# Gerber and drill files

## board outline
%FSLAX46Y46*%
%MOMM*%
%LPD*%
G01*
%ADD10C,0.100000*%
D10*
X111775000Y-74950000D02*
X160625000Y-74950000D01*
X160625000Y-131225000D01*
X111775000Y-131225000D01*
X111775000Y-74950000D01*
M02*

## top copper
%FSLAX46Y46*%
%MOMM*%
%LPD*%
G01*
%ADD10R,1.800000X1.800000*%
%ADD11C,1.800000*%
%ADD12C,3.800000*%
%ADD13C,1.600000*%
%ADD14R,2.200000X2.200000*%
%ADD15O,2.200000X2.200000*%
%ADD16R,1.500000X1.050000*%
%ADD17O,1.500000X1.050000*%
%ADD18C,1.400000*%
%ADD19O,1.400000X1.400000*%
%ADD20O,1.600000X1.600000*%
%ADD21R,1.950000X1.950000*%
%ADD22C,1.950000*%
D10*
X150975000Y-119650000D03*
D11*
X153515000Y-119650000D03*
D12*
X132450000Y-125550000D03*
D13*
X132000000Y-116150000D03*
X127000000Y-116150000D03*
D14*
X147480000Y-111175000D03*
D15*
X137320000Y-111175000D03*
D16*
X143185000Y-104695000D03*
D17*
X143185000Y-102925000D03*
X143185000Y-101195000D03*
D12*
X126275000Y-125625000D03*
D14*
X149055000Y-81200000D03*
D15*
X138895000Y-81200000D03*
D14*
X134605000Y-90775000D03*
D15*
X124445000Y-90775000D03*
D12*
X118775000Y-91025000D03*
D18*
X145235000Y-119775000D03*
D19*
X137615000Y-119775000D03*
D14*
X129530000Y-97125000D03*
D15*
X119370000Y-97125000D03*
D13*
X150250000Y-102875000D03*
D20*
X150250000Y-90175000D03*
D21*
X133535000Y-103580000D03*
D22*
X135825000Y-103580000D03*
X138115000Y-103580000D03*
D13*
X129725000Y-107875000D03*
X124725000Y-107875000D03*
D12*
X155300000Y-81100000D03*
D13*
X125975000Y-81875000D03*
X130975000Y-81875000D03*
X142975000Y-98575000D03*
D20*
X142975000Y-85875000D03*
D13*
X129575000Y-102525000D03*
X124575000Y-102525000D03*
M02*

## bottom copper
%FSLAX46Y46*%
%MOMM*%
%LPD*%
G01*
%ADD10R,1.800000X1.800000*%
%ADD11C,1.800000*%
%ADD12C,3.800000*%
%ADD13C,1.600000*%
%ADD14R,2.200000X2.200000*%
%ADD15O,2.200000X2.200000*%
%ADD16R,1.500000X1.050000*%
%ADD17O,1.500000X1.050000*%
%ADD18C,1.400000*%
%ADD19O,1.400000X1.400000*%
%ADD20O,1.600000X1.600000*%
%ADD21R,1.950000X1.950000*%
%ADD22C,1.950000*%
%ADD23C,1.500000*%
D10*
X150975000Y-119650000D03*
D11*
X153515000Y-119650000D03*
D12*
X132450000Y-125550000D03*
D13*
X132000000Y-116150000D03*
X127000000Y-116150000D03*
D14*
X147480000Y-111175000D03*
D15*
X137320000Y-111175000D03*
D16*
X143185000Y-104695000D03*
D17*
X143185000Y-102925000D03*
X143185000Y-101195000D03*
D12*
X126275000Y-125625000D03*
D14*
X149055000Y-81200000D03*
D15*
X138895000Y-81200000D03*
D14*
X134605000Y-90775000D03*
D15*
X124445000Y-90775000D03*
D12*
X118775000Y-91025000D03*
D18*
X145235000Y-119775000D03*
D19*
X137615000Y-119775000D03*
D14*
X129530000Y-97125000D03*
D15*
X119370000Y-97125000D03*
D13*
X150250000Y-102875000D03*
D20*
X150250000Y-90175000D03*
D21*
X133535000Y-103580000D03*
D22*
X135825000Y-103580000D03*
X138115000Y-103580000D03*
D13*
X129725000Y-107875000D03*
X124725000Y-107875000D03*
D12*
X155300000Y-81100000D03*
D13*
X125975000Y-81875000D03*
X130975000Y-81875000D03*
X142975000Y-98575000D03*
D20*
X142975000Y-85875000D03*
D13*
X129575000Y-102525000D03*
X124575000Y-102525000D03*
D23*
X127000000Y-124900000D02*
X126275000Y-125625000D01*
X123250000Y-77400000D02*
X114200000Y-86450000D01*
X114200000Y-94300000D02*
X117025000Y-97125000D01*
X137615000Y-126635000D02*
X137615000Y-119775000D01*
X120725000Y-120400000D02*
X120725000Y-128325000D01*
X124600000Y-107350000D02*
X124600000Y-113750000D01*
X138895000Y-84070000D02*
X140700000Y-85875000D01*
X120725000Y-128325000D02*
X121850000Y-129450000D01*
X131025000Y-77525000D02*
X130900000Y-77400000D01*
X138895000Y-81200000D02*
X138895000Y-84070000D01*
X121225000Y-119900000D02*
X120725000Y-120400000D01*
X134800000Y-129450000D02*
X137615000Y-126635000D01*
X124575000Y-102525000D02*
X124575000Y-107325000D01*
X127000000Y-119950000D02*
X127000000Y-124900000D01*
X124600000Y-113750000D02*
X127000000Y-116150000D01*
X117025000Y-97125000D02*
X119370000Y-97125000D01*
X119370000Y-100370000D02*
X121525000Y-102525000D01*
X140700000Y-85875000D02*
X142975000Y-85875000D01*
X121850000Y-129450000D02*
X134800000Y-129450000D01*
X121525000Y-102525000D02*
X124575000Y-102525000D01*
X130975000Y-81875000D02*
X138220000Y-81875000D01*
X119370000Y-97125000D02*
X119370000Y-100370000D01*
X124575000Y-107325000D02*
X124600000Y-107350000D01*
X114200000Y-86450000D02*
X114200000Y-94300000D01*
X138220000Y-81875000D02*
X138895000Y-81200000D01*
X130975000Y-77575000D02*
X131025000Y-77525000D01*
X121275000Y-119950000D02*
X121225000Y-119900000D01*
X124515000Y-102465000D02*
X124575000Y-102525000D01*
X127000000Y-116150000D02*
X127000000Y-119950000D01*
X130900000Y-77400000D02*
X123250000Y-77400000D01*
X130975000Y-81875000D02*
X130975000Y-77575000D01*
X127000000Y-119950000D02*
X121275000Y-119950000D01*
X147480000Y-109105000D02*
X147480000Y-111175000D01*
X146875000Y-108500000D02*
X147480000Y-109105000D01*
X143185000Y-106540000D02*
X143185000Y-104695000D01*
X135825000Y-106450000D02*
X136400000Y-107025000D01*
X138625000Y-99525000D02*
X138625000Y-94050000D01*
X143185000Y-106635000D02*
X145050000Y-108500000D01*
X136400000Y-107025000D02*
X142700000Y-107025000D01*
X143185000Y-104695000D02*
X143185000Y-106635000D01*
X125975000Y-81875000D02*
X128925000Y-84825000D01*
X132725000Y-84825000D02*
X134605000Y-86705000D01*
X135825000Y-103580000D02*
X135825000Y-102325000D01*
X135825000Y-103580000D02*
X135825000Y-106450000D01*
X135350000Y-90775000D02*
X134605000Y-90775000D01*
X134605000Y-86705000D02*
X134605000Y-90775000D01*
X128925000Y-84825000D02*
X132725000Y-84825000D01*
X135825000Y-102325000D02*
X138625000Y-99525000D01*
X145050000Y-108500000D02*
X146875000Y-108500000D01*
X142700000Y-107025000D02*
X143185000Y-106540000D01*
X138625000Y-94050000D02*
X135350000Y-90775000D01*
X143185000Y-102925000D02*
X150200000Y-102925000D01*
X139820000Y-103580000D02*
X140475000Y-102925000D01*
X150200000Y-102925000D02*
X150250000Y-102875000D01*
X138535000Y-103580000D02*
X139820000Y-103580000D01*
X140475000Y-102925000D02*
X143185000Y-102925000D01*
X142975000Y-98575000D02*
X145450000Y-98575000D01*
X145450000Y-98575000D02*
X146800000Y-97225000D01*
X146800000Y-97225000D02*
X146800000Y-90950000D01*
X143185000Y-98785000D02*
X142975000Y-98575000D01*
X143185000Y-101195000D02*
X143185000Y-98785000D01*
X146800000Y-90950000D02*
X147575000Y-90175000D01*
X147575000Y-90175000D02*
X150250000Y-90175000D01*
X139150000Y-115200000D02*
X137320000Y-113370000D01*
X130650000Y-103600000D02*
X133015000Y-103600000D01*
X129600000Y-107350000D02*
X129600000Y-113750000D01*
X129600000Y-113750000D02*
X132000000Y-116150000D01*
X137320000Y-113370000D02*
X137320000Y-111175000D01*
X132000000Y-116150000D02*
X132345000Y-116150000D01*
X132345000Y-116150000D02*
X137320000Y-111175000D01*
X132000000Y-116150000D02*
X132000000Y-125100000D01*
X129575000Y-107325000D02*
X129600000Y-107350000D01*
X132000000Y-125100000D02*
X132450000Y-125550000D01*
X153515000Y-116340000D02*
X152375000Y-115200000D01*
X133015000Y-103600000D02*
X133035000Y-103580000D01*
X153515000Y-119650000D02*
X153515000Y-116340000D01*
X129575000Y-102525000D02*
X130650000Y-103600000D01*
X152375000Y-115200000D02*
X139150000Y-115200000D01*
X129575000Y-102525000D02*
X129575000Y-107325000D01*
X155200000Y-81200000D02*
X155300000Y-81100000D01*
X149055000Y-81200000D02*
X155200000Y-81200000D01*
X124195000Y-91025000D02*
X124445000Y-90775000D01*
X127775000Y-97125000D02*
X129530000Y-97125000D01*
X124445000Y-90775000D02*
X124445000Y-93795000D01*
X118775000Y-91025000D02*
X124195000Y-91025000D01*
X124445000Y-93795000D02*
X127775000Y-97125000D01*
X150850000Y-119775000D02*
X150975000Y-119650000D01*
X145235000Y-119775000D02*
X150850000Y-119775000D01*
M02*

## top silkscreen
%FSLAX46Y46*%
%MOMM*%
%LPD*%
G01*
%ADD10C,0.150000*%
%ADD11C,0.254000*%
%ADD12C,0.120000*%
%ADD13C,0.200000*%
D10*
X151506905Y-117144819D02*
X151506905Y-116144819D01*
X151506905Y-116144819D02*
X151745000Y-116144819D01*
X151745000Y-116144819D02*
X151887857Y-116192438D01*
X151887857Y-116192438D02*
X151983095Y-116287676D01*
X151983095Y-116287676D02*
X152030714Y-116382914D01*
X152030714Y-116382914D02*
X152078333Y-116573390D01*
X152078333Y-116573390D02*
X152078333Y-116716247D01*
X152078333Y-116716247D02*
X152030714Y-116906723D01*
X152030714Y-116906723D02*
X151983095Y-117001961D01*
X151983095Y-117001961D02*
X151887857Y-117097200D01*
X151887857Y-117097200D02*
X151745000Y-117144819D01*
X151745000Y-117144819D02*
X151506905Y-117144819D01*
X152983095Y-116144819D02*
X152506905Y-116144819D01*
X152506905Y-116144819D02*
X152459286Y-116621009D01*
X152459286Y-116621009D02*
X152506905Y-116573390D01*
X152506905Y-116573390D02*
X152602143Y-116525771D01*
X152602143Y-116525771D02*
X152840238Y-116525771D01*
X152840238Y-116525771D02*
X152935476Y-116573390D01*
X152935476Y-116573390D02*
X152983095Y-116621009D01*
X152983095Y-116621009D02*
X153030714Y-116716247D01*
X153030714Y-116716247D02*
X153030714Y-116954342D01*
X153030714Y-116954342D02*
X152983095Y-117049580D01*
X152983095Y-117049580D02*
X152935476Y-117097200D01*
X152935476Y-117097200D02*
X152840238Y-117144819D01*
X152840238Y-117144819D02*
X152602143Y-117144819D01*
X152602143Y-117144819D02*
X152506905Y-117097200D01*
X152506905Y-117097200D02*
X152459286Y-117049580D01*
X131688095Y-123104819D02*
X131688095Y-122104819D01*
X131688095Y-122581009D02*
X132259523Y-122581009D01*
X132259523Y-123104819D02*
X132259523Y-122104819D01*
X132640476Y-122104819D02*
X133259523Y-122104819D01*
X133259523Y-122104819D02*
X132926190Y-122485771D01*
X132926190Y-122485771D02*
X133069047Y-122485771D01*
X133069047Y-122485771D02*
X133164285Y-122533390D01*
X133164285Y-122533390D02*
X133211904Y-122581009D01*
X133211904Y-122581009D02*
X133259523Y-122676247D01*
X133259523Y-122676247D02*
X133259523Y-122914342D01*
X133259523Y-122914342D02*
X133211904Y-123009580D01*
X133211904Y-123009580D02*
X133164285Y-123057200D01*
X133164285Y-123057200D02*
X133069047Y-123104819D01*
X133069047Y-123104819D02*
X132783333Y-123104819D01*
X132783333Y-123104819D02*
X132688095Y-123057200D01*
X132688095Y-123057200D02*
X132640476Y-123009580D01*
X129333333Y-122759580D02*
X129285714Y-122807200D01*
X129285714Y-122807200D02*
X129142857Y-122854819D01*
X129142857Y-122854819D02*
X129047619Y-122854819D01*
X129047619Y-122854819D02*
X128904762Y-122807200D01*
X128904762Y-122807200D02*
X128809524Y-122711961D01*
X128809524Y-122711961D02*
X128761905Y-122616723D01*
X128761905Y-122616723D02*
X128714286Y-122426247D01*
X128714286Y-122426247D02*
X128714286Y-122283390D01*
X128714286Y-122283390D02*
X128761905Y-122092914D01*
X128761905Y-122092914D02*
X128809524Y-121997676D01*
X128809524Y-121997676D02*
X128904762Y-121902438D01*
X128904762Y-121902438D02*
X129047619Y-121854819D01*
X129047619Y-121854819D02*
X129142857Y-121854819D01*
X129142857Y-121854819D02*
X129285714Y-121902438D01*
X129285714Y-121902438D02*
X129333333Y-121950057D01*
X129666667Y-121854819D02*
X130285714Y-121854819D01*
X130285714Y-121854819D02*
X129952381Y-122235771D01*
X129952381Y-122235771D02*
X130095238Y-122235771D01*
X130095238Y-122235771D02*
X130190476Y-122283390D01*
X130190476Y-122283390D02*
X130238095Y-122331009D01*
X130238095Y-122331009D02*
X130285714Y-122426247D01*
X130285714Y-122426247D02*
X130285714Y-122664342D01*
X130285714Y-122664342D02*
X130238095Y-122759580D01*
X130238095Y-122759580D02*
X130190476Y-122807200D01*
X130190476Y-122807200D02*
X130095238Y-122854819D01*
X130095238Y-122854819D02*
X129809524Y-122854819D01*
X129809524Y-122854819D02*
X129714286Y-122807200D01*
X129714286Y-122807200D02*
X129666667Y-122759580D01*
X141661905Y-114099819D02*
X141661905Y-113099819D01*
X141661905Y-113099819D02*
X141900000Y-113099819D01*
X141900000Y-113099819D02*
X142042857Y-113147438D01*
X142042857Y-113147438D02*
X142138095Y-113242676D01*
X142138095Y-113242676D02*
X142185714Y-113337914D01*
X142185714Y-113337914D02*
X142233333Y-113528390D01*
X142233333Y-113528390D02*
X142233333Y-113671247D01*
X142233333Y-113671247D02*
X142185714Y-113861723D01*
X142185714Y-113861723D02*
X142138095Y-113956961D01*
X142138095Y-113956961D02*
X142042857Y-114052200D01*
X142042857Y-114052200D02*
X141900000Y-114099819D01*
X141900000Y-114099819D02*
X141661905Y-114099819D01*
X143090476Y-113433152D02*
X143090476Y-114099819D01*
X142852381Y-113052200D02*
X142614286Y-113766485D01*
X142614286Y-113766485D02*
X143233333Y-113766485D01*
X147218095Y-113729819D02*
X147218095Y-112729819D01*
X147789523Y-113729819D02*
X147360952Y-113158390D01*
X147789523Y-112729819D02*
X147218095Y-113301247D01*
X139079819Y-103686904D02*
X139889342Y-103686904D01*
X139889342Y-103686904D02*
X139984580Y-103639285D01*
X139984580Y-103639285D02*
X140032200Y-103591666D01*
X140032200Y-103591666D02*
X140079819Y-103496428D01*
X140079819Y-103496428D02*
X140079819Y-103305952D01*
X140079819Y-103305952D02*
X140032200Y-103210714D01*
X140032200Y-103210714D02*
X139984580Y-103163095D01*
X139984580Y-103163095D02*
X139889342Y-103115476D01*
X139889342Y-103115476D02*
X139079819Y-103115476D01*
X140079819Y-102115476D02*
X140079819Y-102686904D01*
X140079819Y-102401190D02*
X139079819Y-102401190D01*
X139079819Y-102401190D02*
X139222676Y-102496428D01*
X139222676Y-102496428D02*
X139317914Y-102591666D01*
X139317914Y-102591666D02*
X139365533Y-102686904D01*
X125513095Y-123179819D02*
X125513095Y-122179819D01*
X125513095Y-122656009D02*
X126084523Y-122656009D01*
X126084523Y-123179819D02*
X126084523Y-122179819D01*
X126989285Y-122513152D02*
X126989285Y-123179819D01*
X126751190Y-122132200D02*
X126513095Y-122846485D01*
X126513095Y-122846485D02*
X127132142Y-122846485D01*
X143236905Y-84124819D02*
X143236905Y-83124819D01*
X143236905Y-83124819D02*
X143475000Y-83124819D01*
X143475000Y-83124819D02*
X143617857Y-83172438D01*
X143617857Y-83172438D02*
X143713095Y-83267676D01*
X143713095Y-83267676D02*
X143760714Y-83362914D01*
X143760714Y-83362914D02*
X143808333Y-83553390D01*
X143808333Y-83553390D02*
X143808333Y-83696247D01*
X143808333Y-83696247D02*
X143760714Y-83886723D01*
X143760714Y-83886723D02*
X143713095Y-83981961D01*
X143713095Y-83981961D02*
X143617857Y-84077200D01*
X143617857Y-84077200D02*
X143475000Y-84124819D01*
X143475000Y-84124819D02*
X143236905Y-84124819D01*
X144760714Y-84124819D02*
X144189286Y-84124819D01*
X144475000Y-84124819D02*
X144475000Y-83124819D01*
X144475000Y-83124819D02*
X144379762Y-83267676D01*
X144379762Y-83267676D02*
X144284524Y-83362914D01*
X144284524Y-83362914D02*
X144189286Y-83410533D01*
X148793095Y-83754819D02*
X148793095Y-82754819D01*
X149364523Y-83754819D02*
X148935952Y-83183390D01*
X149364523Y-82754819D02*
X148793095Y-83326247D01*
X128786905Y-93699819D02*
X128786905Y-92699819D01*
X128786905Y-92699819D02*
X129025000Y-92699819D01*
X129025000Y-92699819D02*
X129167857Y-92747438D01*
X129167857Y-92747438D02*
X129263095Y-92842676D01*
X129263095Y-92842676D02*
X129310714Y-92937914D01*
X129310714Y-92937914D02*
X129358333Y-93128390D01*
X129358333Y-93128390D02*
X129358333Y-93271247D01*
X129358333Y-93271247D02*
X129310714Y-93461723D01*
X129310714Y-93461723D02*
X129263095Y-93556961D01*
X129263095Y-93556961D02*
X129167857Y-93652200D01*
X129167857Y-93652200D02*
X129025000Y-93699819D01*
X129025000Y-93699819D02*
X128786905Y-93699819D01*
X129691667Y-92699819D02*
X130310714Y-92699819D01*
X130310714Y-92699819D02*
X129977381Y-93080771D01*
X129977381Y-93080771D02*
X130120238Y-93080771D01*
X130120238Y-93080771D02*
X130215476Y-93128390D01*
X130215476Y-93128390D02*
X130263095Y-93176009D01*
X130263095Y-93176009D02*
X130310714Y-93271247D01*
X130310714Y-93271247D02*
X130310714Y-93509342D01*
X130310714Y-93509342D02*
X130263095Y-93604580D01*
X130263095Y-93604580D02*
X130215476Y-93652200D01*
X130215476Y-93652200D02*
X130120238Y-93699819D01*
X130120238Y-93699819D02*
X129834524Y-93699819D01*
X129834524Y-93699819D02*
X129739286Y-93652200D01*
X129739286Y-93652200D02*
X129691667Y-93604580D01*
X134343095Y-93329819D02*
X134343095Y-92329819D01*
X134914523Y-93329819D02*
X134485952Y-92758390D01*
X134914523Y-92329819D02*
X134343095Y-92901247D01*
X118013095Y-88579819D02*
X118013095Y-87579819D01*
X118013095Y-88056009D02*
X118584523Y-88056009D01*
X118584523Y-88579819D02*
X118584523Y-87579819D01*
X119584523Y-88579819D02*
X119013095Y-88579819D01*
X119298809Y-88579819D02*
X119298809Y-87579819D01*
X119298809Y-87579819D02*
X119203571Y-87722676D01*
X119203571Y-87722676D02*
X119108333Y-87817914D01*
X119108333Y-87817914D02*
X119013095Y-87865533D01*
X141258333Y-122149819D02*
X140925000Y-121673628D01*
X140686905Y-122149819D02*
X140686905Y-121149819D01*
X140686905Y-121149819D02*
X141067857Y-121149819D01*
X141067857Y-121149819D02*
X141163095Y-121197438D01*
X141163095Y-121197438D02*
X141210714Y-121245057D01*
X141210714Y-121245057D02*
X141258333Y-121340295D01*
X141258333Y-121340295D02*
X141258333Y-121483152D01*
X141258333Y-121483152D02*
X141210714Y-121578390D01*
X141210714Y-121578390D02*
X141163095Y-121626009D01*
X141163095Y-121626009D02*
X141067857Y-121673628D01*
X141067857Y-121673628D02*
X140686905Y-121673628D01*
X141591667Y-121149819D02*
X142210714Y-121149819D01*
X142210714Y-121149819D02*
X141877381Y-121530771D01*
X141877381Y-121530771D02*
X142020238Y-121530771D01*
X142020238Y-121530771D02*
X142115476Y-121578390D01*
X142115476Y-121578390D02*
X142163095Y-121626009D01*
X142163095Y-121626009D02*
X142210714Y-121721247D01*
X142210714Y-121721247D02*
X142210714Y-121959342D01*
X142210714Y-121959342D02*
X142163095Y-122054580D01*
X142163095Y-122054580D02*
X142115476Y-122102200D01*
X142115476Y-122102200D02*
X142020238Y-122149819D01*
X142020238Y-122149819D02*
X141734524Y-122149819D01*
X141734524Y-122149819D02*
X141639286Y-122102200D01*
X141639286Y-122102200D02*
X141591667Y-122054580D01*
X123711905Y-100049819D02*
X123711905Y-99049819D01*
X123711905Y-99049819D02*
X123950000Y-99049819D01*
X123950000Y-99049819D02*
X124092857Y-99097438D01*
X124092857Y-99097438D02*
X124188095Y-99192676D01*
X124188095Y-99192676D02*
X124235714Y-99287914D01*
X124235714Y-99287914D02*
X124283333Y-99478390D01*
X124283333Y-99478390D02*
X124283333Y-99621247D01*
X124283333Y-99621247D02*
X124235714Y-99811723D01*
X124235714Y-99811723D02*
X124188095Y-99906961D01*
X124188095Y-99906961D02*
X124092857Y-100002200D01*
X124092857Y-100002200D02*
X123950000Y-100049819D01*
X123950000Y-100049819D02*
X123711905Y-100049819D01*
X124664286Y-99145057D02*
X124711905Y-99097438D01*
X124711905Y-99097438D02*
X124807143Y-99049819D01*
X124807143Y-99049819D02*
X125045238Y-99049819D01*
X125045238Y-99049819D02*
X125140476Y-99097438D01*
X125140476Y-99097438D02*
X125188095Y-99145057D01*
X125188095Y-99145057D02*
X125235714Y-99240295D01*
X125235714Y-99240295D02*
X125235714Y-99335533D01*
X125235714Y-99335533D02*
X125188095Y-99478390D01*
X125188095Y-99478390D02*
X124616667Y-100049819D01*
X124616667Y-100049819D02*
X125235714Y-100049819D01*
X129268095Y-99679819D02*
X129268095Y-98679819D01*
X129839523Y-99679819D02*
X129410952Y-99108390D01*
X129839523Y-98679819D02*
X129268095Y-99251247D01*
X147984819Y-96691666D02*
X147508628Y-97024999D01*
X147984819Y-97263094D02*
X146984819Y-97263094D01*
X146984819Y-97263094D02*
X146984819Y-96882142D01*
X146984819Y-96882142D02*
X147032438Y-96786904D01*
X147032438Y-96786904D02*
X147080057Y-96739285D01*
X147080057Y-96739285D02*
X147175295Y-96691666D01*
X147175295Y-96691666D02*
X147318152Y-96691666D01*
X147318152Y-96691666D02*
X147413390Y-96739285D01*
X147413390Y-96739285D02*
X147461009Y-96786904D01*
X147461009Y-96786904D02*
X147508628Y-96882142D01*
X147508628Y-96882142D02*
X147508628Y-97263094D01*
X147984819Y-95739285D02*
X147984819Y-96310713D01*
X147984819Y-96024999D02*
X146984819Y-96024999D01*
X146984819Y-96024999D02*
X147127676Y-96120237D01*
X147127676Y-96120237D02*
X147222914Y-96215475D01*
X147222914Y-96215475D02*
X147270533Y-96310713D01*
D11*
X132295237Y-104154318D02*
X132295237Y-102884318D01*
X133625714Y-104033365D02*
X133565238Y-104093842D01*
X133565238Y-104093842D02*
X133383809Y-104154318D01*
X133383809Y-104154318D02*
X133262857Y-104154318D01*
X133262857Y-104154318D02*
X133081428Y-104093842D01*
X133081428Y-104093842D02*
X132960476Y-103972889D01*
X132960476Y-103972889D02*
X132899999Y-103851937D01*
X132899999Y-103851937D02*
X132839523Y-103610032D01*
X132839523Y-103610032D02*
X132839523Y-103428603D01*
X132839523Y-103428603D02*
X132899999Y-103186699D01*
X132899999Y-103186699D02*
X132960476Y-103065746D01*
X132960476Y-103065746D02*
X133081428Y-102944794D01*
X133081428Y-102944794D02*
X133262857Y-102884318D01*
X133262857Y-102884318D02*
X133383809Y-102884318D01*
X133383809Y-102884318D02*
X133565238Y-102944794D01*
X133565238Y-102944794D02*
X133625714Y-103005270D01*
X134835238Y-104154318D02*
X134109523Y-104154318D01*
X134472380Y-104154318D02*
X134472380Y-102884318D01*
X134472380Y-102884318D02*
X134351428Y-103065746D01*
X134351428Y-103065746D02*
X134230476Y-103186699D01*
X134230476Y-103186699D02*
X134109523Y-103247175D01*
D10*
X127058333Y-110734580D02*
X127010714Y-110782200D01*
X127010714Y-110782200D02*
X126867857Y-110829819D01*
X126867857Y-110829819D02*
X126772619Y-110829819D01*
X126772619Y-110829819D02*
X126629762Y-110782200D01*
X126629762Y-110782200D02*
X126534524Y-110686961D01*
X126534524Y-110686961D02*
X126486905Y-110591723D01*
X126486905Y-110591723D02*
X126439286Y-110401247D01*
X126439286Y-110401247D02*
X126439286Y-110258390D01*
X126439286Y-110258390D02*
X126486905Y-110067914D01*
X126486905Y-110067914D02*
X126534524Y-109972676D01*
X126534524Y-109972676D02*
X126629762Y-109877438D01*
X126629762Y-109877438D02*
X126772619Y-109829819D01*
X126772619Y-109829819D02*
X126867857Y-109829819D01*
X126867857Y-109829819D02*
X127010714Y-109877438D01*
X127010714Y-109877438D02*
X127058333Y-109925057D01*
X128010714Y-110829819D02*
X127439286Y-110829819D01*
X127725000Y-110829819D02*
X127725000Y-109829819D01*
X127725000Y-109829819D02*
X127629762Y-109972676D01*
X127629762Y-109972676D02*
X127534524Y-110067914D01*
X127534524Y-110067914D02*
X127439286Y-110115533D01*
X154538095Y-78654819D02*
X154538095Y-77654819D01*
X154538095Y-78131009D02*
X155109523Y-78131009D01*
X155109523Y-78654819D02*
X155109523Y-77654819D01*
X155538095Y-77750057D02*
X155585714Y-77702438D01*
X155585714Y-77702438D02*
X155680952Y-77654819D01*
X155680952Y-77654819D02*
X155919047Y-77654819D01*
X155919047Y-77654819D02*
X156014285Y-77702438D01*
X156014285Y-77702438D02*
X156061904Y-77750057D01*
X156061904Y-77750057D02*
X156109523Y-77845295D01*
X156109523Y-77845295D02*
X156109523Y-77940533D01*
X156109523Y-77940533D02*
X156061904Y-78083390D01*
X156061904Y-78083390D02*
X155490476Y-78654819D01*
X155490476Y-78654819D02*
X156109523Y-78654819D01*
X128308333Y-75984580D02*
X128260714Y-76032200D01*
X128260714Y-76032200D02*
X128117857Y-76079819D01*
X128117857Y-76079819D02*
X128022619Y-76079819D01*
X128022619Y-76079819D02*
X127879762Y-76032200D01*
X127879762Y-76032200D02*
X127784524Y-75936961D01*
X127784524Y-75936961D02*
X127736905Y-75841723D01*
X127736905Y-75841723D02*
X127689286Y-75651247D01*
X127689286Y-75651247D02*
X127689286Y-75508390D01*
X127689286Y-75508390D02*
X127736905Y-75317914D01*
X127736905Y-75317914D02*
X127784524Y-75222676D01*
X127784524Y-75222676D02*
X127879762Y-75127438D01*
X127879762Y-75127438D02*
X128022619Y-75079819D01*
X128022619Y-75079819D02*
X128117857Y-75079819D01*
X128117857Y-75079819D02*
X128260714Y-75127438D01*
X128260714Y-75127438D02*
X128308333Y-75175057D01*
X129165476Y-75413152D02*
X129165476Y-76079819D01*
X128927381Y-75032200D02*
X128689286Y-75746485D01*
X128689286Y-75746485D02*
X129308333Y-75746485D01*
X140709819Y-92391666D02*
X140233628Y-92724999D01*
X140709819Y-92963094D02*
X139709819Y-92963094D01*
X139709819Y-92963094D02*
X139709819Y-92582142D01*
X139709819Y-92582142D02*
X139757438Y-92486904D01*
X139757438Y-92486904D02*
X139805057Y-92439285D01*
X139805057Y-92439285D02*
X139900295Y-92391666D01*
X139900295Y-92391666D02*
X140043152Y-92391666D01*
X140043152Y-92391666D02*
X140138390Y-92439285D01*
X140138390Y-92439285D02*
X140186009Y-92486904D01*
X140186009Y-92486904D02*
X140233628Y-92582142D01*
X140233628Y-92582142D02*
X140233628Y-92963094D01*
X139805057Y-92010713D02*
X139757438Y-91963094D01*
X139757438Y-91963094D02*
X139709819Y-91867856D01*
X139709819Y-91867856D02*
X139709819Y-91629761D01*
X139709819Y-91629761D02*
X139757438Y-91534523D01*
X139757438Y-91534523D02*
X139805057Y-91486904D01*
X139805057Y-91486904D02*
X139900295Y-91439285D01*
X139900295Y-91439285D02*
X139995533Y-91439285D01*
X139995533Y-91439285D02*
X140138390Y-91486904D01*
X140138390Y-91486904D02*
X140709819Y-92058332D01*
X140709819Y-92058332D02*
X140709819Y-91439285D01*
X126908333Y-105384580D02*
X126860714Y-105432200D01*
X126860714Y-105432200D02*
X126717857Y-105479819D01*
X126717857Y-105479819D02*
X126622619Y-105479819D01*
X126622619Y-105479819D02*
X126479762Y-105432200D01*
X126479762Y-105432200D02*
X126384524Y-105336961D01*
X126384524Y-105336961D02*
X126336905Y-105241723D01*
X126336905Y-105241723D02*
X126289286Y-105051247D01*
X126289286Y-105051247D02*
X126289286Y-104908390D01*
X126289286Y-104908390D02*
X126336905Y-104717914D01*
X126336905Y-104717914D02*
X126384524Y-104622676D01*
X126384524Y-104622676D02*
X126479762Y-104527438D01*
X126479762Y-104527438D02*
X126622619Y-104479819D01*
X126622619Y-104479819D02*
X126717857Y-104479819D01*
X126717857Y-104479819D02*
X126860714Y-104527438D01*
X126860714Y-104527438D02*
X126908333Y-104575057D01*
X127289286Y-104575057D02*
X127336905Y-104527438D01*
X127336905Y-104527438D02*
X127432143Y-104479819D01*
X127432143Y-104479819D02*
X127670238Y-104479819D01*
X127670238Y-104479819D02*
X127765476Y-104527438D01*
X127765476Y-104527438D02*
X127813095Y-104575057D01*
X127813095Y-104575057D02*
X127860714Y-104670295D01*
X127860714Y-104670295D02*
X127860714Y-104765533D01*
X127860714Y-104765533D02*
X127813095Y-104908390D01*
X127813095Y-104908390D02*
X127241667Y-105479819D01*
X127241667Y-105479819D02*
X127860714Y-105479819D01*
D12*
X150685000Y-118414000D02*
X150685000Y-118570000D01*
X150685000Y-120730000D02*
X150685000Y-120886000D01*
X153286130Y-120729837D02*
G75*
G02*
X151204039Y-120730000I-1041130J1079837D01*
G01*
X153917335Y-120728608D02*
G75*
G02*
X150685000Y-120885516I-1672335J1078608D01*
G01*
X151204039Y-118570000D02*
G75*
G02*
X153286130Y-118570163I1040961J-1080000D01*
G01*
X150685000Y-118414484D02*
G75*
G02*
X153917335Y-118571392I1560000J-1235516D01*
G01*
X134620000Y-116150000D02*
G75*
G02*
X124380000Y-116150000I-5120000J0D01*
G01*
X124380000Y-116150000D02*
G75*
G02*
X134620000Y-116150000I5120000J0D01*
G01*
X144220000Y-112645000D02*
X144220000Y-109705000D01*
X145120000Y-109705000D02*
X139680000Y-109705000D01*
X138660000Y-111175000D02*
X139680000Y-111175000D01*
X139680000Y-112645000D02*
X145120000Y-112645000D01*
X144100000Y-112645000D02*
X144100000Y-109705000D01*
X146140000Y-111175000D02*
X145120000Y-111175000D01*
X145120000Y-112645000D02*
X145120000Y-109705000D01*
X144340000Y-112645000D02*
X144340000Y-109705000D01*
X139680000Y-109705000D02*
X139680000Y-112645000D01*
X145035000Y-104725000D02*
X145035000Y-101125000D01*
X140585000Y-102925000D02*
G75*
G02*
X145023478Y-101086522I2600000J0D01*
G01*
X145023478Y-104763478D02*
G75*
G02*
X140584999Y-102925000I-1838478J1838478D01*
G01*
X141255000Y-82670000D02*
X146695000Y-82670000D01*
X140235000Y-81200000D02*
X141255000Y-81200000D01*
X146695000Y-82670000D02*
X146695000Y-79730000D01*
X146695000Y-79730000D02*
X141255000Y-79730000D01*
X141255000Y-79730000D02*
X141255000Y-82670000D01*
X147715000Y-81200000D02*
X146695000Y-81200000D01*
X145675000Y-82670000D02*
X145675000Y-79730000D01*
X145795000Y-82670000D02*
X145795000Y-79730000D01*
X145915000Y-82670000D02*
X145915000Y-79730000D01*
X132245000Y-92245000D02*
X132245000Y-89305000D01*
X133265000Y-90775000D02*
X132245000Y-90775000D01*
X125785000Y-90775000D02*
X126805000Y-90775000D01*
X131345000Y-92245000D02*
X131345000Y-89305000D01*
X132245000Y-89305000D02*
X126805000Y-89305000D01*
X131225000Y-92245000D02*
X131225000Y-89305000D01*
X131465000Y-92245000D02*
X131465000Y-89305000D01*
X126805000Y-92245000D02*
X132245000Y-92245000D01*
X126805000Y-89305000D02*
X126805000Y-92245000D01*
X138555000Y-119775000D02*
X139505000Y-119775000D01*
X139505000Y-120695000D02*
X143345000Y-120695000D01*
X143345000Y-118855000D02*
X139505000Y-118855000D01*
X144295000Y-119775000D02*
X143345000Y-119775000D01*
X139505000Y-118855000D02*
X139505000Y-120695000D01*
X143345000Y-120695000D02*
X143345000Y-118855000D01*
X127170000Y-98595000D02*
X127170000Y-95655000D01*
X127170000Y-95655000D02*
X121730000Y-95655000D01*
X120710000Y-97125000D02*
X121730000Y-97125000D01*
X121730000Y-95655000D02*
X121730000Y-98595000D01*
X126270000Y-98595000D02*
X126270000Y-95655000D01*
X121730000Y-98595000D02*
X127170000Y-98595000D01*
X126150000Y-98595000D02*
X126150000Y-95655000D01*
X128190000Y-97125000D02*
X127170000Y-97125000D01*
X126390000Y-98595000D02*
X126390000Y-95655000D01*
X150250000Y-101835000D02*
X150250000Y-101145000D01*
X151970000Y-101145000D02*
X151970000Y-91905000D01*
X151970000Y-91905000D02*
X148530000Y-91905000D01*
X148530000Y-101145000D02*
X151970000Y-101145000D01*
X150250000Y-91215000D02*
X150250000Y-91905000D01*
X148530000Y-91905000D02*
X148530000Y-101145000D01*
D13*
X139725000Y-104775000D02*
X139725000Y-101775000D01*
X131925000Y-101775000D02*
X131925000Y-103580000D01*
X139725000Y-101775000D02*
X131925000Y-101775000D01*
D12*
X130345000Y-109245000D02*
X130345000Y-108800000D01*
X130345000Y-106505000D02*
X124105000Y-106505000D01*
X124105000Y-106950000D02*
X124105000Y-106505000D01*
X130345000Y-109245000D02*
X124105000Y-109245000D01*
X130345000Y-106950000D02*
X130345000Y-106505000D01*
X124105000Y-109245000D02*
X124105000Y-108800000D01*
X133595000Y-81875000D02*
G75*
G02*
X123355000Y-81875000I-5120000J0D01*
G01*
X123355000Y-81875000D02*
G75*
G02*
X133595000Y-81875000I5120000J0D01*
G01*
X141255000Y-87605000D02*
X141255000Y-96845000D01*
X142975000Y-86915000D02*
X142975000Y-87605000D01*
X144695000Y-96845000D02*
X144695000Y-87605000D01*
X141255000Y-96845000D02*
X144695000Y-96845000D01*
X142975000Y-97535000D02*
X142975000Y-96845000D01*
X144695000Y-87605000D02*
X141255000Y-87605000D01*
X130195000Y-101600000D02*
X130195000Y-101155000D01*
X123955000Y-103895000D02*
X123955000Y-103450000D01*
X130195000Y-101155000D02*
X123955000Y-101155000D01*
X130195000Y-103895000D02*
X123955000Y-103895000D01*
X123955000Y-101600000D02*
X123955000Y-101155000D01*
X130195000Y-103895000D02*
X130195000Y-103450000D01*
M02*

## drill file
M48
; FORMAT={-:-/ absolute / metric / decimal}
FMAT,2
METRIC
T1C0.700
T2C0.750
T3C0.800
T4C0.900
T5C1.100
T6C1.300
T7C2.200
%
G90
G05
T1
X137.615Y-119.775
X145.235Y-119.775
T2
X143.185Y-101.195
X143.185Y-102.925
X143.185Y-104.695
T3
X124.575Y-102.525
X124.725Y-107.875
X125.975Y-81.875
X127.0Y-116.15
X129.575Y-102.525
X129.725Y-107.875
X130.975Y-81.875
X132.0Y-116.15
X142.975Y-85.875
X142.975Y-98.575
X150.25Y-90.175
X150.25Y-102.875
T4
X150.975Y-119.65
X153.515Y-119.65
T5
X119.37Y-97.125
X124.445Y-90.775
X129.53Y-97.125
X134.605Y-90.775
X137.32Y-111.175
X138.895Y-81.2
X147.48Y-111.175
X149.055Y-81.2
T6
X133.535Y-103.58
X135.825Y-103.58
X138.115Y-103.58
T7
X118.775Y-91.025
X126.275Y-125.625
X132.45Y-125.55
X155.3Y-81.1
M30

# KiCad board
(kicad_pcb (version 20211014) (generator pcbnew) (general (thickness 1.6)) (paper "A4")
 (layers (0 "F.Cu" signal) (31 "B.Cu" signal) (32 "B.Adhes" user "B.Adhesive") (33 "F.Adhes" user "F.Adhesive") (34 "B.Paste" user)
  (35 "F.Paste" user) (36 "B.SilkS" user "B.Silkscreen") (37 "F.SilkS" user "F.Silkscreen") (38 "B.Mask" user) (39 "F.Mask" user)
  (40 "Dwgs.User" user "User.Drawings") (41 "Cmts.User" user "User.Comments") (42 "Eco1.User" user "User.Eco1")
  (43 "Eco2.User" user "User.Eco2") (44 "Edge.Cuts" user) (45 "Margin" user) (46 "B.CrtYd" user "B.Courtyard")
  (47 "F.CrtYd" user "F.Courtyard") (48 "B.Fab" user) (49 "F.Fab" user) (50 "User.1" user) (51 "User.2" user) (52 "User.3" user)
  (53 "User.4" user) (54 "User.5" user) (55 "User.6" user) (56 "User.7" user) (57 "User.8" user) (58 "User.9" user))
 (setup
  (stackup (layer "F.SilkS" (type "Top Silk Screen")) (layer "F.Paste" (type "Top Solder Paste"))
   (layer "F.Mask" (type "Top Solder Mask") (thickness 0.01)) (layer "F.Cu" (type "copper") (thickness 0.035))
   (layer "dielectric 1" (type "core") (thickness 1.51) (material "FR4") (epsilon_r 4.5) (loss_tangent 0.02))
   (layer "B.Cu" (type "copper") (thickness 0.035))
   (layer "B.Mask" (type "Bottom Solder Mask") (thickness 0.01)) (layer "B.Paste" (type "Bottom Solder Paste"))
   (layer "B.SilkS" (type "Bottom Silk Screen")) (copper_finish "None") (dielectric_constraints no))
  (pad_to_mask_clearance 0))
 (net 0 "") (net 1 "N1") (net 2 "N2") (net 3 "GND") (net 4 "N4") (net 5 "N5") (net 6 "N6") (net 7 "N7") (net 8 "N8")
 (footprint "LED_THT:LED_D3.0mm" (layer "F.Cu") (at 150.975 119.65)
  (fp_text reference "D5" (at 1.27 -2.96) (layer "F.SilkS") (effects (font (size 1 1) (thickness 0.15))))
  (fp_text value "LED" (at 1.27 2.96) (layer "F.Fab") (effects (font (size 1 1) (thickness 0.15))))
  (fp_line (start -0.29 -1.236) (end -0.29 -1.08) (layer "F.SilkS") (width 0.12))
  (fp_line (start -0.29 1.08) (end -0.29 1.236) (layer "F.SilkS") (width 0.12))
  (fp_arc (start 2.31113 1.079837) (mid 1.270117 1.5) (end 0.229039 1.08) (layer "F.SilkS") (width 0.12))
  (fp_arc (start 2.942335 1.078608) (mid 1.366487 1.987659) (end -0.29 1.235516) (layer "F.SilkS") (width 0.12))
  (fp_arc (start 0.229039 -1.08) (mid 1.270117 -1.5) (end 2.31113 -1.079837) (layer "F.SilkS") (width 0.12))
  (fp_arc (start -0.29 -1.235516) (mid 1.366487 -1.987659) (end 2.942335 -1.078608) (layer "F.SilkS") (width 0.12))
  (pad "1" thru_hole rect (at 0 0) (size 1.8 1.8) (drill 0.9) (layers *.Cu *.Mask) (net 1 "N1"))
  (pad "2" thru_hole circle (at 2.54 0) (size 1.8 1.8) (drill 0.9) (layers *.Cu *.Mask) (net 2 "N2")))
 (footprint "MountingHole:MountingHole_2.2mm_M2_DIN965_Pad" (layer "F.Cu") (at 132.45 125.55)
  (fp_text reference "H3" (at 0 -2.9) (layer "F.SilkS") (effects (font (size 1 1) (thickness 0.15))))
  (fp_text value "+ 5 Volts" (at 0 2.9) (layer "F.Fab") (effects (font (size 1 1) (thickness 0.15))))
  (pad "1" thru_hole circle (at 0 0) (size 3.8 3.8) (drill 2.2) (layers *.Cu *.Mask) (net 2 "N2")))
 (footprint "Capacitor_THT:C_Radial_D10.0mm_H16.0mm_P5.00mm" (layer "F.Cu") (at 132 116.15 180)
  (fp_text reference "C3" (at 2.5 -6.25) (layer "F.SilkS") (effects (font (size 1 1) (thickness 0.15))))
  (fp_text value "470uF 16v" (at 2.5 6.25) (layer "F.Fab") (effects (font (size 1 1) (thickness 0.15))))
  (fp_circle (center 2.5 0) (end 7.62 0) (layer "F.SilkS") (width 0.12) (fill none))
  (pad "1" thru_hole circle (at 0 0 180) (size 1.6 1.6) (drill 0.8) (layers *.Cu *.Mask) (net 2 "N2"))
  (pad "2" thru_hole circle (at 5 0 180) (size 1.6 1.6) (drill 0.8) (layers *.Cu *.Mask) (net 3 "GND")))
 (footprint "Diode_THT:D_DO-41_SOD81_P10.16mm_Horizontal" (layer "F.Cu") (at 147.48 111.175 180)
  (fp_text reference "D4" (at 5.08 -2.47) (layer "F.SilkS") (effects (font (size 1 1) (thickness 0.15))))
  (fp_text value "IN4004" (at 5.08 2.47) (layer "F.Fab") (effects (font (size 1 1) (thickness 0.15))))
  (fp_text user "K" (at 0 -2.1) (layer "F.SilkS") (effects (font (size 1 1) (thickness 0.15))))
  (fp_line (start 3.26 -1.47) (end 3.26 1.47) (layer "F.SilkS") (width 0.12))
  (fp_line (start 2.36 1.47) (end 7.8 1.47) (layer "F.SilkS") (width 0.12))
  (fp_line (start 8.82 0) (end 7.8 0) (layer "F.SilkS") (width 0.12))
  (fp_line (start 7.8 -1.47) (end 2.36 -1.47) (layer "F.SilkS") (width 0.12))
  (fp_line (start 3.38 -1.47) (end 3.38 1.47) (layer "F.SilkS") (width 0.12))
  (fp_line (start 1.34 0) (end 2.36 0) (layer "F.SilkS") (width 0.12))
  (fp_line (start 2.36 -1.47) (end 2.36 1.47) (layer "F.SilkS") (width 0.12))
  (fp_line (start 3.14 -1.47) (end 3.14 1.47) (layer "F.SilkS") (width 0.12))
  (fp_line (start 7.8 1.47) (end 7.8 -1.47) (layer "F.SilkS") (width 0.12))
  (pad "1" thru_hole rect (at 0 0 180) (size 2.2 2.2) (drill 1.1) (layers *.Cu *.Mask) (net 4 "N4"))
  (pad "2" thru_hole oval (at 10.16 0 180) (size 2.2 2.2) (drill 1.1) (layers *.Cu *.Mask) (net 2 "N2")))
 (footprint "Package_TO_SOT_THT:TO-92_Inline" (layer "F.Cu") (at 143.185 104.195 90)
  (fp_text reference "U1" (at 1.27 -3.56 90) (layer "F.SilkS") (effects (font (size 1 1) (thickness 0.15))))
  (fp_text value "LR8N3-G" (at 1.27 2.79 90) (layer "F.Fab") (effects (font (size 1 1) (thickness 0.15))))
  (fp_line (start -0.53 1.85) (end 3.07 1.85) (layer "F.SilkS") (width 0.12))
  (fp_arc (start 1.27 -2.6) (mid 3.672087 -0.994977) (end 3.108478 1.838478) (layer "F.SilkS") (width 0.12))
  (fp_arc (start -0.568478 1.838478) (mid -1.132087 -0.994977) (end 1.27 -2.6) (layer "F.SilkS") (width 0.12))
  (pad "1" thru_hole rect (at -0.5 0 90) (size 1.05 1.5) (drill 0.75) (layers *.Cu *.Mask) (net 4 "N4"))
  (pad "2" thru_hole oval (at 1.27 0 90) (size 1.05 1.5) (drill 0.75) (layers *.Cu *.Mask) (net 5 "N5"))
  (pad "3" thru_hole oval (at 3 0 90) (size 1.05 1.5) (drill 0.75) (layers *.Cu *.Mask) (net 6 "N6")))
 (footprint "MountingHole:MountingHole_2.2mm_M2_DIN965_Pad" (layer "F.Cu") (at 126.275 125.625)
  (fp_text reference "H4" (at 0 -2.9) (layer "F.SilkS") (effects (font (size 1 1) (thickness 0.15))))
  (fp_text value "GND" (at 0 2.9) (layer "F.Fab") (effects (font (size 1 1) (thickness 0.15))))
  (pad "1" thru_hole circle (at 0 0) (size 3.8 3.8) (drill 2.2) (layers *.Cu *.Mask) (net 3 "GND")))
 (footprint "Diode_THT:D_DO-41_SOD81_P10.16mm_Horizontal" (layer "F.Cu") (at 149.055 81.2 180)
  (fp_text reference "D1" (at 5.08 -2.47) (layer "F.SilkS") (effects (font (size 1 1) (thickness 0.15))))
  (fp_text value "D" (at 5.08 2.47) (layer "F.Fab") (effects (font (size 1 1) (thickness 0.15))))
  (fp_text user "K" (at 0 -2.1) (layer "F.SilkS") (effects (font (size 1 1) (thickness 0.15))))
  (fp_line (start 7.8 -1.47) (end 2.36 -1.47) (layer "F.SilkS") (width 0.12))
  (fp_line (start 8.82 0) (end 7.8 0) (layer "F.SilkS") (width 0.12))
  (fp_line (start 2.36 -1.47) (end 2.36 1.47) (layer "F.SilkS") (width 0.12))
  (fp_line (start 2.36 1.47) (end 7.8 1.47) (layer "F.SilkS") (width 0.12))
  (fp_line (start 7.8 1.47) (end 7.8 -1.47) (layer "F.SilkS") (width 0.12))
  (fp_line (start 1.34 0) (end 2.36 0) (layer "F.SilkS") (width 0.12))
  (fp_line (start 3.38 -1.47) (end 3.38 1.47) (layer "F.SilkS") (width 0.12))
  (fp_line (start 3.26 -1.47) (end 3.26 1.47) (layer "F.SilkS") (width 0.12))
  (fp_line (start 3.14 -1.47) (end 3.14 1.47) (layer "F.SilkS") (width 0.12))
  (pad "1" thru_hole rect (at 0 0 180) (size 2.2 2.2) (drill 1.1) (layers *.Cu *.Mask) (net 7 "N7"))
  (pad "2" thru_hole oval (at 10.16 0 180) (size 2.2 2.2) (drill 1.1) (layers *.Cu *.Mask) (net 3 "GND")))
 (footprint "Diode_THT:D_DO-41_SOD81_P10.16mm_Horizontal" (layer "F.Cu") (at 134.605 90.775 180)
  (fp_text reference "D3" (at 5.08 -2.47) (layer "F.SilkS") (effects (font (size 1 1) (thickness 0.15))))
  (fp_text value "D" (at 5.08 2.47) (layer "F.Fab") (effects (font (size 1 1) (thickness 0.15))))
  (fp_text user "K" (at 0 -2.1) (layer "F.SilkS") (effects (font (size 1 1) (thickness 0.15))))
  (fp_line (start 2.36 -1.47) (end 2.36 1.47) (layer "F.SilkS") (width 0.12))
  (fp_line (start 1.34 0) (end 2.36 0) (layer "F.SilkS") (width 0.12))
  (fp_line (start 8.82 0) (end 7.8 0) (layer "F.SilkS") (width 0.12))
  (fp_line (start 3.26 -1.47) (end 3.26 1.47) (layer "F.SilkS") (width 0.12))
  (fp_line (start 2.36 1.47) (end 7.8 1.47) (layer "F.SilkS") (width 0.12))
  (fp_line (start 3.38 -1.47) (end 3.38 1.47) (layer "F.SilkS") (width 0.12))
  (fp_line (start 3.14 -1.47) (end 3.14 1.47) (layer "F.SilkS") (width 0.12))
  (fp_line (start 7.8 -1.47) (end 2.36 -1.47) (layer "F.SilkS") (width 0.12))
  (fp_line (start 7.8 1.47) (end 7.8 -1.47) (layer "F.SilkS") (width 0.12))
  (pad "1" thru_hole rect (at 0 0 180) (size 2.2 2.2) (drill 1.1) (layers *.Cu *.Mask) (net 4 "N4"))
  (pad "2" thru_hole oval (at 10.16 0 180) (size 2.2 2.2) (drill 1.1) (layers *.Cu *.Mask) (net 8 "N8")))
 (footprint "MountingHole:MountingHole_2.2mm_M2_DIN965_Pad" (layer "F.Cu") (at 118.775 91.025)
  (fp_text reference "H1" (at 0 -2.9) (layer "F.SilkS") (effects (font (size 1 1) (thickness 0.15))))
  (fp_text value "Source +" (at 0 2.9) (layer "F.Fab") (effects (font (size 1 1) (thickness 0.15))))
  (pad "1" thru_hole circle (at 0 0) (size 3.8 3.8) (drill 2.2) (layers *.Cu *.Mask) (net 8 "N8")))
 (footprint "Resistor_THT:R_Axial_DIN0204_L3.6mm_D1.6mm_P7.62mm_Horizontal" (layer "F.Cu") (at 145.235 119.775 180)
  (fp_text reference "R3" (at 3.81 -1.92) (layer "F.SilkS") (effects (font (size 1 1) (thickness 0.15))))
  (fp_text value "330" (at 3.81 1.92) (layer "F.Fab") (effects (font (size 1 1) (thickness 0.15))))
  (fp_line (start 6.68 0) (end 5.73 0) (layer "F.SilkS") (width 0.12))
  (fp_line (start 5.73 -0.92) (end 1.89 -0.92) (layer "F.SilkS") (width 0.12))
  (fp_line (start 1.89 0.92) (end 5.73 0.92) (layer "F.SilkS") (width 0.12))
  (fp_line (start 0.94 0) (end 1.89 0) (layer "F.SilkS") (width 0.12))
  (fp_line (start 5.73 0.92) (end 5.73 -0.92) (layer "F.SilkS") (width 0.12))
  (fp_line (start 1.89 -0.92) (end 1.89 0.92) (layer "F.SilkS") (width 0.12))
  (pad "1" thru_hole circle (at 0 0 180) (size 1.4 1.4) (drill 0.7) (layers *.Cu *.Mask) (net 1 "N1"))
  (pad "2" thru_hole oval (at 7.62 0 180) (size 1.4 1.4) (drill 0.7) (layers *.Cu *.Mask) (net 3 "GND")))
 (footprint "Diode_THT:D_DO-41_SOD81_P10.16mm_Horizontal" (layer "F.Cu") (at 129.53 97.125 180)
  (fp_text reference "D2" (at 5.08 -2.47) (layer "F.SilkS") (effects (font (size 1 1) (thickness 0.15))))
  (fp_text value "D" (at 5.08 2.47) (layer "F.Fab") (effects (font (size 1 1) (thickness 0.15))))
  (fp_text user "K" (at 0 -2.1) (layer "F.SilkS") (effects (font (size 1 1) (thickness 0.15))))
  (fp_line (start 2.36 -1.47) (end 2.36 1.47) (layer "F.SilkS") (width 0.12))
  (fp_line (start 2.36 1.47) (end 7.8 1.47) (layer "F.SilkS") (width 0.12))
  (fp_line (start 8.82 0) (end 7.8 0) (layer "F.SilkS") (width 0.12))
  (fp_line (start 7.8 1.47) (end 7.8 -1.47) (layer "F.SilkS") (width 0.12))
  (fp_line (start 3.26 -1.47) (end 3.26 1.47) (layer "F.SilkS") (width 0.12))
  (fp_line (start 7.8 -1.47) (end 2.36 -1.47) (layer "F.SilkS") (width 0.12))
  (fp_line (start 3.38 -1.47) (end 3.38 1.47) (layer "F.SilkS") (width 0.12))
  (fp_line (start 1.34 0) (end 2.36 0) (layer "F.SilkS") (width 0.12))
  (fp_line (start 3.14 -1.47) (end 3.14 1.47) (layer "F.SilkS") (width 0.12))
  (pad "1" thru_hole rect (at 0 0 180) (size 2.2 2.2) (drill 1.1) (layers *.Cu *.Mask) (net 8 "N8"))
  (pad "2" thru_hole oval (at 10.16 0 180) (size 2.2 2.2) (drill 1.1) (layers *.Cu *.Mask) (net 3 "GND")))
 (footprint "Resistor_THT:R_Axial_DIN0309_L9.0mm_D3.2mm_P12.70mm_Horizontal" (layer "F.Cu") (at 150.25 102.875 90)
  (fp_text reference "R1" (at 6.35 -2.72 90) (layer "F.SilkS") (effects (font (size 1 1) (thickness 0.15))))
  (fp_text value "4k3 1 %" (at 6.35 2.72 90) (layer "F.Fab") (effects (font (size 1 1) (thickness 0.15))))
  (fp_line (start 1.04 0) (end 1.73 0) (layer "F.SilkS") (width 0.12))
  (fp_line (start 1.73 1.72) (end 10.97 1.72) (layer "F.SilkS") (width 0.12))
  (fp_line (start 10.97 1.72) (end 10.97 -1.72) (layer "F.SilkS") (width 0.12))
  (fp_line (start 1.73 -1.72) (end 1.73 1.72) (layer "F.SilkS") (width 0.12))
  (fp_line (start 11.66 0) (end 10.97 0) (layer "F.SilkS") (width 0.12))
  (fp_line (start 10.97 -1.72) (end 1.73 -1.72) (layer "F.SilkS") (width 0.12))
  (pad "1" thru_hole circle (at 0 0 90) (size 1.6 1.6) (drill 0.8) (layers *.Cu *.Mask) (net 5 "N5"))
  (pad "2" thru_hole oval (at 12.7 0 90) (size 1.6 1.6) (drill 0.8) (layers *.Cu *.Mask) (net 6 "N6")))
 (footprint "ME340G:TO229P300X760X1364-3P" (layer "F.Cu") (at 133.535 103.58)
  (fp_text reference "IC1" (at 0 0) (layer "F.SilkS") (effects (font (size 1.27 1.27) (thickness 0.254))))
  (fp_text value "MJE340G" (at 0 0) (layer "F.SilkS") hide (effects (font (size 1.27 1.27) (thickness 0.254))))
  (fp_line (start 6.19 1.195) (end 6.19 -1.805) (layer "F.SilkS") (width 0.2))
  (fp_line (start -1.61 -1.805) (end -1.61 0) (layer "F.SilkS") (width 0.2))
  (fp_line (start 6.19 -1.805) (end -1.61 -1.805) (layer "F.SilkS") (width 0.2))
  (pad "1" thru_hole rect locked (at 0 0) (size 1.95 1.95) (drill 1.3) (layers *.Cu *.Mask) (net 2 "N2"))
  (pad "2" thru_hole circle locked (at 2.29 0) (size 1.95 1.95) (drill 1.3) (layers *.Cu *.Mask) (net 4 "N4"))
  (pad "3" thru_hole circle locked (at 4.58 0) (size 1.95 1.95) (drill 1.3) (layers *.Cu *.Mask) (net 5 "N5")))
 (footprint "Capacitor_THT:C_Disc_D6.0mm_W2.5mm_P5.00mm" (layer "F.Cu") (at 129.725 107.875 180)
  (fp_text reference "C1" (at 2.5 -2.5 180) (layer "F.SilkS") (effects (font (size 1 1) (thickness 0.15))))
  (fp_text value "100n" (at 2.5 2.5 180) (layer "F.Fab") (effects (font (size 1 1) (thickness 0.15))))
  (fp_line (start -0.62 -1.37) (end -0.62 -0.925) (layer "F.SilkS") (width 0.12))
  (fp_line (start -0.62 1.37) (end 5.62 1.37) (layer "F.SilkS") (width 0.12))
  (fp_line (start 5.62 0.925) (end 5.62 1.37) (layer "F.SilkS") (width 0.12))
  (fp_line (start -0.62 -1.37) (end 5.62 -1.37) (layer "F.SilkS") (width 0.12))
  (fp_line (start -0.62 0.925) (end -0.62 1.37) (layer "F.SilkS") (width 0.12))
  (fp_line (start 5.62 -1.37) (end 5.62 -0.925) (layer "F.SilkS") (width 0.12))
  (pad "1" thru_hole circle (at 0 0 180) (size 1.6 1.6) (drill 0.8) (layers *.Cu *.Mask) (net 2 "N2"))
  (pad "2" thru_hole circle (at 5 0 180) (size 1.6 1.6) (drill 0.8) (layers *.Cu *.Mask) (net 3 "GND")))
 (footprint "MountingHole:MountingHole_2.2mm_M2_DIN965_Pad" (layer "F.Cu") (at 155.3 81.1)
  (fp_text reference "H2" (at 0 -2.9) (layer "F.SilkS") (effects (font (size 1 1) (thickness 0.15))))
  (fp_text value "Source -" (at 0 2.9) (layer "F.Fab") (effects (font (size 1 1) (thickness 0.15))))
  (pad "1" thru_hole circle (at 0 0) (size 3.8 3.8) (drill 2.2) (layers *.Cu *.Mask) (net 7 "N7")))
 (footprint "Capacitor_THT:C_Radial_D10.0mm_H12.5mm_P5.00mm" (layer "F.Cu") (at 125.975 81.875)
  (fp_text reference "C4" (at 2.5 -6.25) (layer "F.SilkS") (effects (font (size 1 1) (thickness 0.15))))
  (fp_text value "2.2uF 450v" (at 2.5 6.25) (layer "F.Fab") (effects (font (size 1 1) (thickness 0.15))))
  (fp_circle (center 2.5 0) (end 7.62 0) (layer "F.SilkS") (width 0.12) (fill none))
  (pad "1" thru_hole circle (at 0 0) (size 1.6 1.6) (drill 0.8) (layers *.Cu *.Mask) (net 4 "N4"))
  (pad "2" thru_hole circle (at 5 0) (size 1.6 1.6) (drill 0.8) (layers *.Cu *.Mask) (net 3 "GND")))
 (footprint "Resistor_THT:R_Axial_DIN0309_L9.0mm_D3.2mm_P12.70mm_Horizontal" (layer "F.Cu") (at 142.975 98.575 90)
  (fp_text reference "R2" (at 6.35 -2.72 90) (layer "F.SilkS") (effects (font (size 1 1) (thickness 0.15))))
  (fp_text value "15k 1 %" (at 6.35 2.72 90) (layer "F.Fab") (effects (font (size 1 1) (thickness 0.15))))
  (fp_line (start 10.97 -1.72) (end 1.73 -1.72) (layer "F.SilkS") (width 0.12))
  (fp_line (start 11.66 0) (end 10.97 0) (layer "F.SilkS") (width 0.12))
  (fp_line (start 1.73 1.72) (end 10.97 1.72) (layer "F.SilkS") (width 0.12))
  (fp_line (start 1.73 -1.72) (end 1.73 1.72) (layer "F.SilkS") (width 0.12))
  (fp_line (start 1.04 0) (end 1.73 0) (layer "F.SilkS") (width 0.12))
  (fp_line (start 10.97 1.72) (end 10.97 -1.72) (layer "F.SilkS") (width 0.12))
  (pad "1" thru_hole circle (at 0 0 90) (size 1.6 1.6) (drill 0.8) (layers *.Cu *.Mask) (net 6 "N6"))
  (pad "2" thru_hole oval (at 12.7 0 90) (size 1.6 1.6) (drill 0.8) (layers *.Cu *.Mask) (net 3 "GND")))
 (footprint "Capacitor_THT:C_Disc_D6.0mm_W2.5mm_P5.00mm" (layer "F.Cu") (at 129.575 102.525 180)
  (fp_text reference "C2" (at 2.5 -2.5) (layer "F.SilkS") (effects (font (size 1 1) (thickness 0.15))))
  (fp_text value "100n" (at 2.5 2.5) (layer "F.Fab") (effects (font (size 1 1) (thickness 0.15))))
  (fp_line (start -0.62 0.925) (end -0.62 1.37) (layer "F.SilkS") (width 0.12))
  (fp_line (start 5.62 -1.37) (end 5.62 -0.925) (layer "F.SilkS") (width 0.12))
  (fp_line (start -0.62 1.37) (end 5.62 1.37) (layer "F.SilkS") (width 0.12))
  (fp_line (start -0.62 -1.37) (end 5.62 -1.37) (layer "F.SilkS") (width 0.12))
  (fp_line (start 5.62 0.925) (end 5.62 1.37) (layer "F.SilkS") (width 0.12))
  (fp_line (start -0.62 -1.37) (end -0.62 -0.925) (layer "F.SilkS") (width 0.12))
  (pad "1" thru_hole circle (at 0 0 180) (size 1.6 1.6) (drill 0.8) (layers *.Cu *.Mask) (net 2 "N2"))
  (pad "2" thru_hole circle (at 5 0 180) (size 1.6 1.6) (drill 0.8) (layers *.Cu *.Mask) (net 3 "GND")))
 (gr_rect (start 111.775 74.95) (end 160.625 131.225) (layer "Edge.Cuts") (width 0.1) (fill none))
 (segment (start 127 124.9) (end 126.275 125.625) (width 1.5) (layer "B.Cu") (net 3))
 (segment (start 123.25 77.4) (end 114.2 86.45) (width 1.5) (layer "B.Cu") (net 3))
 (segment (start 114.2 94.3) (end 117.025 97.125) (width 1.5) (layer "B.Cu") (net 3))
 (segment (start 137.615 126.635) (end 137.615 119.775) (width 1.5) (layer "B.Cu") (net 3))
 (segment (start 120.725 120.4) (end 120.725 128.325) (width 1.5) (layer "B.Cu") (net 3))
 (segment (start 124.6 107.35) (end 124.6 113.75) (width 1.5) (layer "B.Cu") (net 3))
 (segment (start 138.895 84.07) (end 140.7 85.875) (width 1.5) (layer "B.Cu") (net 3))
 (segment (start 120.725 128.325) (end 121.85 129.45) (width 1.5) (layer "B.Cu") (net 3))
 (segment (start 131.025 77.525) (end 130.9 77.4) (width 1.5) (layer "B.Cu") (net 3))
 (segment (start 138.895 81.2) (end 138.895 84.07) (width 1.5) (layer "B.Cu") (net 3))
 (segment (start 121.225 119.9) (end 120.725 120.4) (width 1.5) (layer "B.Cu") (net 3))
 (segment (start 134.8 129.45) (end 137.615 126.635) (width 1.5) (layer "B.Cu") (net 3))
 (segment (start 124.575 102.525) (end 124.575 107.325) (width 1.5) (layer "B.Cu") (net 3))
 (segment (start 127 119.95) (end 127 124.9) (width 1.5) (layer "B.Cu") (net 3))
 (segment (start 124.6 113.75) (end 127 116.15) (width 1.5) (layer "B.Cu") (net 3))
 (segment (start 117.025 97.125) (end 119.37 97.125) (width 1.5) (layer "B.Cu") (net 3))
 (segment (start 119.37 100.37) (end 121.525 102.525) (width 1.5) (layer "B.Cu") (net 3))
 (segment (start 140.7 85.875) (end 142.975 85.875) (width 1.5) (layer "B.Cu") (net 3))
 (segment (start 121.85 129.45) (end 134.8 129.45) (width 1.5) (layer "B.Cu") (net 3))
 (segment (start 121.525 102.525) (end 124.575 102.525) (width 1.5) (layer "B.Cu") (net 3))
 (segment (start 130.975 81.875) (end 138.22 81.875) (width 1.5) (layer "B.Cu") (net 3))
 (segment (start 119.37 97.125) (end 119.37 100.37) (width 1.5) (layer "B.Cu") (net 3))
 (segment (start 124.575 107.325) (end 124.6 107.35) (width 1.5) (layer "B.Cu") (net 3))
 (segment (start 114.2 86.45) (end 114.2 94.3) (width 1.5) (layer "B.Cu") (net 3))
 (segment (start 138.22 81.875) (end 138.895 81.2) (width 1.5) (layer "B.Cu") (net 3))
 (segment (start 130.975 77.575) (end 131.025 77.525) (width 1.5) (layer "B.Cu") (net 3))
 (segment (start 121.275 119.95) (end 121.225 119.9) (width 1.5) (layer "B.Cu") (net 3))
 (segment (start 124.515 102.465) (end 124.575 102.525) (width 1.5) (layer "B.Cu") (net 3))
 (segment (start 127 116.15) (end 127 119.95) (width 1.5) (layer "B.Cu") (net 3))
 (segment (start 130.9 77.4) (end 123.25 77.4) (width 1.5) (layer "B.Cu") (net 3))
 (segment (start 130.975 81.875) (end 130.975 77.575) (width 1.5) (layer "B.Cu") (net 3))
 (segment (start 127 119.95) (end 121.275 119.95) (width 1.5) (layer "B.Cu") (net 3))
 (segment (start 147.48 109.105) (end 147.48 111.175) (width 1.5) (layer "B.Cu") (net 4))
 (segment (start 146.875 108.5) (end 147.48 109.105) (width 1.5) (layer "B.Cu") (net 4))
 (segment (start 143.185 106.54) (end 143.185 104.695) (width 1.5) (layer "B.Cu") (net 4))
 (segment (start 135.825 106.45) (end 136.4 107.025) (width 1.5) (layer "B.Cu") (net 4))
 (segment (start 138.625 99.525) (end 138.625 94.05) (width 1.5) (layer "B.Cu") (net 4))
 (segment (start 143.185 106.635) (end 145.05 108.5) (width 1.5) (layer "B.Cu") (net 4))
 (segment (start 136.4 107.025) (end 142.7 107.025) (width 1.5) (layer "B.Cu") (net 4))
 (segment (start 143.185 104.695) (end 143.185 106.635) (width 1.5) (layer "B.Cu") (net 4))
 (segment (start 125.975 81.875) (end 128.925 84.825) (width 1.5) (layer "B.Cu") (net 4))
 (segment (start 132.725 84.825) (end 134.605 86.705) (width 1.5) (layer "B.Cu") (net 4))
 (segment (start 135.825 103.58) (end 135.825 102.325) (width 1.5) (layer "B.Cu") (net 4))
 (segment (start 135.825 103.58) (end 135.825 106.45) (width 1.5) (layer "B.Cu") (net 4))
 (segment (start 135.35 90.775) (end 134.605 90.775) (width 1.5) (layer "B.Cu") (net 4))
 (segment (start 134.605 86.705) (end 134.605 90.775) (width 1.5) (layer "B.Cu") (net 4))
 (segment (start 128.925 84.825) (end 132.725 84.825) (width 1.5) (layer "B.Cu") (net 4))
 (segment (start 135.825 102.325) (end 138.625 99.525) (width 1.5) (layer "B.Cu") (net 4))
 (segment (start 145.05 108.5) (end 146.875 108.5) (width 1.5) (layer "B.Cu") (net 4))
 (segment (start 142.7 107.025) (end 143.185 106.54) (width 1.5) (layer "B.Cu") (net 4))
 (segment (start 138.625 94.05) (end 135.35 90.775) (width 1.5) (layer "B.Cu") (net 4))
 (segment (start 143.185 102.925) (end 150.2 102.925) (width 1.5) (layer "B.Cu") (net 5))
 (segment (start 139.82 103.58) (end 140.475 102.925) (width 1.5) (layer "B.Cu") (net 5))
 (segment (start 150.2 102.925) (end 150.25 102.875) (width 1.5) (layer "B.Cu") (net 5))
 (segment (start 138.535 103.58) (end 139.82 103.58) (width 1.5) (layer "B.Cu") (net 5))
 (segment (start 140.475 102.925) (end 143.185 102.925) (width 1.5) (layer "B.Cu") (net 5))
 (segment (start 142.975 98.575) (end 145.45 98.575) (width 1.5) (layer "B.Cu") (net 6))
 (segment (start 145.45 98.575) (end 146.8 97.225) (width 1.5) (layer "B.Cu") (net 6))
 (segment (start 146.8 97.225) (end 146.8 90.95) (width 1.5) (layer "B.Cu") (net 6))
 (segment (start 143.185 98.785) (end 142.975 98.575) (width 1.5) (layer "B.Cu") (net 6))
 (segment (start 143.185 101.195) (end 143.185 98.785) (width 1.5) (layer "B.Cu") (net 6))
 (segment (start 146.8 90.95) (end 147.575 90.175) (width 1.5) (layer "B.Cu") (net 6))
 (segment (start 147.575 90.175) (end 150.25 90.175) (width 1.5) (layer "B.Cu") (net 6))
 (segment (start 139.15 115.2) (end 137.32 113.37) (width 1.5) (layer "B.Cu") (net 2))
 (segment (start 130.65 103.6) (end 133.015 103.6) (width 1.5) (layer "B.Cu") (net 2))
 (segment (start 129.6 107.35) (end 129.6 113.75) (width 1.5) (layer "B.Cu") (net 2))
 (segment (start 129.6 113.75) (end 132 116.15) (width 1.5) (layer "B.Cu") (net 2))
 (segment (start 137.32 113.37) (end 137.32 111.175) (width 1.5) (layer "B.Cu") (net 2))
 (segment (start 132 116.15) (end 132.345 116.15) (width 1.5) (layer "B.Cu") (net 2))
 (segment (start 132.345 116.15) (end 137.32 111.175) (width 1.5) (layer "B.Cu") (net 2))
 (segment (start 132 116.15) (end 132 125.1) (width 1.5) (layer "B.Cu") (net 2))
 (segment (start 129.575 107.325) (end 129.6 107.35) (width 1.5) (layer "B.Cu") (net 2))
 (segment (start 132 125.1) (end 132.45 125.55) (width 1.5) (layer "B.Cu") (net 2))
 (segment (start 153.515 116.34) (end 152.375 115.2) (width 1.5) (layer "B.Cu") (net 2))
 (segment (start 133.015 103.6) (end 133.035 103.58) (width 1.5) (layer "B.Cu") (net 2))
 (segment (start 153.515 119.65) (end 153.515 116.34) (width 1.5) (layer "B.Cu") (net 2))
 (segment (start 129.575 102.525) (end 130.65 103.6) (width 1.5) (layer "B.Cu") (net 2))
 (segment (start 152.375 115.2) (end 139.15 115.2) (width 1.5) (layer "B.Cu") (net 2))
 (segment (start 129.575 102.525) (end 129.575 107.325) (width 1.5) (layer "B.Cu") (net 2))
 (segment (start 155.2 81.2) (end 155.3 81.1) (width 1.5) (layer "B.Cu") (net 7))
 (segment (start 149.055 81.2) (end 155.2 81.2) (width 1.5) (layer "B.Cu") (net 7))
 (segment (start 124.195 91.025) (end 124.445 90.775) (width 1.5) (layer "B.Cu") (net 8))
 (segment (start 127.775 97.125) (end 129.53 97.125) (width 1.5) (layer "B.Cu") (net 8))
 (segment (start 124.445 90.775) (end 124.445 93.795) (width 1.5) (layer "B.Cu") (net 8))
 (segment (start 118.775 91.025) (end 124.195 91.025) (width 1.5) (layer "B.Cu") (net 8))
 (segment (start 124.445 93.795) (end 127.775 97.125) (width 1.5) (layer "B.Cu") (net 8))
 (segment (start 150.85 119.775) (end 150.975 119.65) (width 1.5) (layer "B.Cu") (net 1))
 (segment (start 145.235 119.775) (end 150.85 119.775) (width 1.5) (layer "B.Cu") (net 1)))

